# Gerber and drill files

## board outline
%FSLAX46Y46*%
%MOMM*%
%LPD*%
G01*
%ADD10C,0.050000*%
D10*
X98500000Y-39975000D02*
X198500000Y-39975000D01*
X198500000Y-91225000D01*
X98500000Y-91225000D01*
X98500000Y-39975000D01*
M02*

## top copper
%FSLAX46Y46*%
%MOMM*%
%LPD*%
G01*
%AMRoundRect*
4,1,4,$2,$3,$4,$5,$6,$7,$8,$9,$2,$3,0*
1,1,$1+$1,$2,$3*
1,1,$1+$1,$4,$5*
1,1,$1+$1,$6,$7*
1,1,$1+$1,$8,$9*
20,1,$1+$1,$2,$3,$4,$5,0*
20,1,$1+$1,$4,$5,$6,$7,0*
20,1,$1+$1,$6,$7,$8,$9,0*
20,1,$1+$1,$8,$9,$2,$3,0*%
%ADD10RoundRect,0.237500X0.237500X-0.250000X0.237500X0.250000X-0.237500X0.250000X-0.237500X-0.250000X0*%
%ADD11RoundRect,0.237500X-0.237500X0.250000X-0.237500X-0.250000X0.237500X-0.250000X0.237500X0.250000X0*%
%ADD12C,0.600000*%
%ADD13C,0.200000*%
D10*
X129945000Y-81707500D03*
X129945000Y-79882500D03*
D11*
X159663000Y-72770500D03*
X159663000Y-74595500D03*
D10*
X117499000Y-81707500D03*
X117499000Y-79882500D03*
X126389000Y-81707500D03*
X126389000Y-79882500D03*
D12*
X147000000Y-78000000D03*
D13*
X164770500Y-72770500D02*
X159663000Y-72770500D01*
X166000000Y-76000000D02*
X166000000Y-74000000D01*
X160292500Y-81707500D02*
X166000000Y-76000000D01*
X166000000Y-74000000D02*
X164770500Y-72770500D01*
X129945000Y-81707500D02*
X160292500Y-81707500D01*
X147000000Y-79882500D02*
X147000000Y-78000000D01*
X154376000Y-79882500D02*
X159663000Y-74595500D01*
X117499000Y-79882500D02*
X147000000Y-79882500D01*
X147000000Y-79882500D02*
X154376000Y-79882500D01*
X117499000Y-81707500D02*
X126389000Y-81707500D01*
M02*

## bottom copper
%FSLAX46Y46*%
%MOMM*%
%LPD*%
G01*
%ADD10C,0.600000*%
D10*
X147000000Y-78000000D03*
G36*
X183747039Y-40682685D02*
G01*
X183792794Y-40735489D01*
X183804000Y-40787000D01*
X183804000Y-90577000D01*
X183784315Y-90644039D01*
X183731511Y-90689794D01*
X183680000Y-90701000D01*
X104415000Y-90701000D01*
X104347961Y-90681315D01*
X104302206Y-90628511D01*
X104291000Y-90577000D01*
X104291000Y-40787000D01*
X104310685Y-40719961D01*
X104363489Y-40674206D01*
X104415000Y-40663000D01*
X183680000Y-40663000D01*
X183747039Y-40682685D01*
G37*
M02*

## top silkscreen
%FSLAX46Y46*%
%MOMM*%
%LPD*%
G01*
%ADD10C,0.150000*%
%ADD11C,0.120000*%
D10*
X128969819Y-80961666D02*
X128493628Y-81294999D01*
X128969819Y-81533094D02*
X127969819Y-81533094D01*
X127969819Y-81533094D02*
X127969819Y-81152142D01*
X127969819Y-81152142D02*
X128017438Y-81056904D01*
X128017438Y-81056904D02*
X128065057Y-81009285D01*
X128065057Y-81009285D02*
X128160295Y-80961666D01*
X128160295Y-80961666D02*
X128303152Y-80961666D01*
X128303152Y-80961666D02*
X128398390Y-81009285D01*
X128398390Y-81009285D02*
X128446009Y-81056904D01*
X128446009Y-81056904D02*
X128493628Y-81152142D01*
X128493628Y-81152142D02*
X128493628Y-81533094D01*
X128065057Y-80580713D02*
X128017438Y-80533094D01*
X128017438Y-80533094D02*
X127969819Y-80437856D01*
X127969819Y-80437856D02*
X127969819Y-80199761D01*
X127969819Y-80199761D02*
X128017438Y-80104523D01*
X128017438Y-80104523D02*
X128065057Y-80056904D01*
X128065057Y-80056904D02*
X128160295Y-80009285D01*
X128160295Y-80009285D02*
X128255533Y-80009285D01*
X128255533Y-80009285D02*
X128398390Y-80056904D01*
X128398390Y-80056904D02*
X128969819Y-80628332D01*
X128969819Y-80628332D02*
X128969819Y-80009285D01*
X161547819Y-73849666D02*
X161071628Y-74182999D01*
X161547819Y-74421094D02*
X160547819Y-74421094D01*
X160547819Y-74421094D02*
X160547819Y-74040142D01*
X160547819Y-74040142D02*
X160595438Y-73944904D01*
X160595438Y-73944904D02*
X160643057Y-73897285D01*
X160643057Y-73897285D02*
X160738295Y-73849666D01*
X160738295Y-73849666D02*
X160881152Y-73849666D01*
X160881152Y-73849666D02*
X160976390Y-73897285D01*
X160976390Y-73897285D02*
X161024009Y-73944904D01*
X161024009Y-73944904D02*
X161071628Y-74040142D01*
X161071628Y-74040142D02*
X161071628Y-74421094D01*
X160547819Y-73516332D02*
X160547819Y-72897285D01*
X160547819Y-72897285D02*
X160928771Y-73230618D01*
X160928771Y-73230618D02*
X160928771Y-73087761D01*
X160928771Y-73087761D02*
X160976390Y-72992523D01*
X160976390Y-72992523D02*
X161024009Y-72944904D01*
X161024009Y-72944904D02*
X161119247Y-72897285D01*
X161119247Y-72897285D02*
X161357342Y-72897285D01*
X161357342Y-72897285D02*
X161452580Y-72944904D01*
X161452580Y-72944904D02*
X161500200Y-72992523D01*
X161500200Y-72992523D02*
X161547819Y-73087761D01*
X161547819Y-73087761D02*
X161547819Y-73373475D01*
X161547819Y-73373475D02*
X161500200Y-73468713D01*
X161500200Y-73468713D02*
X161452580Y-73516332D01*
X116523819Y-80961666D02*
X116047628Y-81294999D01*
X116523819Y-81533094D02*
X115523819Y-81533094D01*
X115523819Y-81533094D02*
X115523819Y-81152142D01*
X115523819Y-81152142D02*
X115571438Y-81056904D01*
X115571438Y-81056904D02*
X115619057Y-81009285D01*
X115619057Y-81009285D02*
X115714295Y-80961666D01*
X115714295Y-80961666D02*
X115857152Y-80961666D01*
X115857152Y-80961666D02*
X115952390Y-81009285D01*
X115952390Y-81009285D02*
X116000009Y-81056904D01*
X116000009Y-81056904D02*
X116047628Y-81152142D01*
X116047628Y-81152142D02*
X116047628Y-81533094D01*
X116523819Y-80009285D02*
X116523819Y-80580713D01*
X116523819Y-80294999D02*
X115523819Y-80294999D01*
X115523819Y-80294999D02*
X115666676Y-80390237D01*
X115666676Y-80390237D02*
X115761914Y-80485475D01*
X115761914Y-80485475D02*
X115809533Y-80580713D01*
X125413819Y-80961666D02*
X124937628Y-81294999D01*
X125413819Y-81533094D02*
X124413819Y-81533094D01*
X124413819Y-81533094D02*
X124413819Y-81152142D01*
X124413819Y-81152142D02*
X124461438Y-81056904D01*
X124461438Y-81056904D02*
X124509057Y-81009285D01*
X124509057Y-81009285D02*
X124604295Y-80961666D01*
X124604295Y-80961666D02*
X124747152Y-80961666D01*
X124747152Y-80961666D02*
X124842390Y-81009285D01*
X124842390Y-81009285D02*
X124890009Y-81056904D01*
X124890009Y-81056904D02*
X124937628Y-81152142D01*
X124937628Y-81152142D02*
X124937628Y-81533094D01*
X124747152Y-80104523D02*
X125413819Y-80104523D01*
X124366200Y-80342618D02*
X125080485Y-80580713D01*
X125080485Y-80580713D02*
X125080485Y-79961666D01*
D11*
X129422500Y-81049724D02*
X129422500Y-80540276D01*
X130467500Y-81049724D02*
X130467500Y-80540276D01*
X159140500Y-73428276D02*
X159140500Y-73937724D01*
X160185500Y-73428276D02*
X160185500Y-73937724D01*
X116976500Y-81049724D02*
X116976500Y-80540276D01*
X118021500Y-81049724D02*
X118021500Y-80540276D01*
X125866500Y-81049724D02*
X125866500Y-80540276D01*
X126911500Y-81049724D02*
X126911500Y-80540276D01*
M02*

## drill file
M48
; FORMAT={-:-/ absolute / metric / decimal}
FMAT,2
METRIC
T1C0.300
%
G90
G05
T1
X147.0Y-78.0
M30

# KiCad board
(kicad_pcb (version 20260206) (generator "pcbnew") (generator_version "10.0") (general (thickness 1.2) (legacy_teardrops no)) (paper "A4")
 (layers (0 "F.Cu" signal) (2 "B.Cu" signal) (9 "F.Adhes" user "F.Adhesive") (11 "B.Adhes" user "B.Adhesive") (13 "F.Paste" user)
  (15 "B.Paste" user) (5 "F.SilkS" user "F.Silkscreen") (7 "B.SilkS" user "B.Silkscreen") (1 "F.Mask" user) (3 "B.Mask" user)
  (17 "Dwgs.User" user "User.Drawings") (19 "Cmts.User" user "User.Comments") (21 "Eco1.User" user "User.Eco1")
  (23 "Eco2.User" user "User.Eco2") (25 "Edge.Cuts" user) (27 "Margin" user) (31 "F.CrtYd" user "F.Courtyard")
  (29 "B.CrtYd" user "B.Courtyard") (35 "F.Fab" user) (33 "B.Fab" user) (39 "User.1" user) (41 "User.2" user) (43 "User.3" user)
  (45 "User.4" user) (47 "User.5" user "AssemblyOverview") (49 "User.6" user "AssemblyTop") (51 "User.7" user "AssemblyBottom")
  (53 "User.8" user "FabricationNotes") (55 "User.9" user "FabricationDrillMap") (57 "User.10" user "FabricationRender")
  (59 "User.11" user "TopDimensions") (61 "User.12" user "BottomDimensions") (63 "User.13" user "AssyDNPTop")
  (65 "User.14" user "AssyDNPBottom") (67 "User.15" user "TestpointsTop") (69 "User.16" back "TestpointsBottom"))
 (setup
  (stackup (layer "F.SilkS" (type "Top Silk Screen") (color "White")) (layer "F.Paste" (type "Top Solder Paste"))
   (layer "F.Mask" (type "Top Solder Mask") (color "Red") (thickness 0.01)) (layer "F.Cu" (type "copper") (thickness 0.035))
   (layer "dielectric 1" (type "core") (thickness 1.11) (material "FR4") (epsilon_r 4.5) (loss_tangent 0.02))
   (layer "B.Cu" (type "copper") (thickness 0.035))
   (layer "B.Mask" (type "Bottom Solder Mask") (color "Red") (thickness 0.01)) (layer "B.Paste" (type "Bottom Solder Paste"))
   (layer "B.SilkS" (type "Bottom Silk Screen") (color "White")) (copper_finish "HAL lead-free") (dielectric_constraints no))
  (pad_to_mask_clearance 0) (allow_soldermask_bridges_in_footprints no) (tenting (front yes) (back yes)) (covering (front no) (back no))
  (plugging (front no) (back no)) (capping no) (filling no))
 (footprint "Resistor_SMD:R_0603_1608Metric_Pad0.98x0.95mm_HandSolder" (layer "F.Cu") (at 129.945 80.795 90)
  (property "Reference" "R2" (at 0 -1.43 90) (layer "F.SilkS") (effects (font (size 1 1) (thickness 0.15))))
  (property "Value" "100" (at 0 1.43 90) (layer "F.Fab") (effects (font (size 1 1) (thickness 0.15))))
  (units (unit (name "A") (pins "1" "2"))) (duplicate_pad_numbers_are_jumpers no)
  (fp_line (start -0.254724 -0.5225) (end 0.254724 -0.5225) (stroke (width 0.12) (type solid)) (layer "F.SilkS"))
  (fp_line (start -0.254724 0.5225) (end 0.254724 0.5225) (stroke (width 0.12) (type solid)) (layer "F.SilkS"))
  (pad "1" smd roundrect (at -0.9125 0 90) (size 0.975 0.95) (layers "F.Cu" "F.Mask" "F.Paste") (roundrect_rratio 0.25)
   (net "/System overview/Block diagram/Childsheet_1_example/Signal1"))
  (pad "2" smd roundrect (at 0.9125 0 90) (size 0.975 0.95) (layers "F.Cu" "F.Mask" "F.Paste") (roundrect_rratio 0.25) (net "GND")))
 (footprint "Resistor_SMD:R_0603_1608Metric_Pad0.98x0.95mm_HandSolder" (layer "F.Cu") (at 159.663 73.683 -90)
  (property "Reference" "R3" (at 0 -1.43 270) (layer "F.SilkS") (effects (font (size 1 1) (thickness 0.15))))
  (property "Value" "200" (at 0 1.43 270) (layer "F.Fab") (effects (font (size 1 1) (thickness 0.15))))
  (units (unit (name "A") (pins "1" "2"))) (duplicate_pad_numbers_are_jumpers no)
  (fp_line (start -0.254724 0.5225) (end 0.254724 0.5225) (stroke (width 0.12) (type solid)) (layer "F.SilkS"))
  (fp_line (start -0.254724 -0.5225) (end 0.254724 -0.5225) (stroke (width 0.12) (type solid)) (layer "F.SilkS"))
  (pad "1" smd roundrect (at -0.9125 0 270) (size 0.975 0.95) (layers "F.Cu" "F.Mask" "F.Paste") (roundrect_rratio 0.25)
   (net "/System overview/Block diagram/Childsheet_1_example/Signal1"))
  (pad "2" smd roundrect (at 0.9125 0 270) (size 0.975 0.95) (layers "F.Cu" "F.Mask" "F.Paste") (roundrect_rratio 0.25) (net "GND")))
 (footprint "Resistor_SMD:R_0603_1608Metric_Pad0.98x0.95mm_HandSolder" (layer "F.Cu") (at 117.499 80.795 90)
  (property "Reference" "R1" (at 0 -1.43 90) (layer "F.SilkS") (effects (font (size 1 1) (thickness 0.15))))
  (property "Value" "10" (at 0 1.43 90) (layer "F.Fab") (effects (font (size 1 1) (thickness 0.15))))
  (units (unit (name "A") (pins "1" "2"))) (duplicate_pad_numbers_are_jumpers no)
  (fp_line (start -0.254724 -0.5225) (end 0.254724 -0.5225) (stroke (width 0.12) (type solid)) (layer "F.SilkS"))
  (fp_line (start -0.254724 0.5225) (end 0.254724 0.5225) (stroke (width 0.12) (type solid)) (layer "F.SilkS"))
  (pad "1" smd roundrect (at -0.9125 0 90) (size 0.975 0.95) (layers "F.Cu" "F.Mask" "F.Paste") (roundrect_rratio 0.25)
   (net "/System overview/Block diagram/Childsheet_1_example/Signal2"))
  (pad "2" smd roundrect (at 0.9125 0 90) (size 0.975 0.95) (layers "F.Cu" "F.Mask" "F.Paste") (roundrect_rratio 0.25) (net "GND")))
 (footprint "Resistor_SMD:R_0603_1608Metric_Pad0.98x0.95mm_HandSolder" (layer "F.Cu") (at 126.389 80.795 90)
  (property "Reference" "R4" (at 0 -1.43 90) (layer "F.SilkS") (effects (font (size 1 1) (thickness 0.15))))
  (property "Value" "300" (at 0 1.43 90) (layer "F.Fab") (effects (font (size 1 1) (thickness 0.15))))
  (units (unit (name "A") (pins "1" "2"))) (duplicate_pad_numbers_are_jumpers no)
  (fp_line (start -0.254724 -0.5225) (end 0.254724 -0.5225) (stroke (width 0.12) (type solid)) (layer "F.SilkS"))
  (fp_line (start -0.254724 0.5225) (end 0.254724 0.5225) (stroke (width 0.12) (type solid)) (layer "F.SilkS"))
  (pad "1" smd roundrect (at -0.9125 0 90) (size 0.975 0.95) (layers "F.Cu" "F.Mask" "F.Paste") (roundrect_rratio 0.25)
   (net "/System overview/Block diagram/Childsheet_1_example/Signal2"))
  (pad "2" smd roundrect (at 0.9125 0 90) (size 0.975 0.95) (layers "F.Cu" "F.Mask" "F.Paste") (roundrect_rratio 0.25) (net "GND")))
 (gr_rect (start 98.5 39.975) (end 198.5 91.225) (stroke (width 0.05) (type solid)) (fill no) (layer "Edge.Cuts"))
 (segment (start 164.7705 72.7705) (end 159.663 72.7705) (width 0.2) (layer "F.Cu")
  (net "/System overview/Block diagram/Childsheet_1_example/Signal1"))
 (segment (start 166 76) (end 166 74) (width 0.2) (layer "F.Cu") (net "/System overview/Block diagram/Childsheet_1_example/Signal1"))
 (segment (start 160.2925 81.7075) (end 166 76) (width 0.2) (layer "F.Cu")
  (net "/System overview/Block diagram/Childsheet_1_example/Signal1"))
 (segment (start 166 74) (end 164.7705 72.7705) (width 0.2) (layer "F.Cu")
  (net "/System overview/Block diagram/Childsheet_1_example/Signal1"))
 (segment (start 129.945 81.7075) (end 160.2925 81.7075) (width 0.2) (layer "F.Cu")
  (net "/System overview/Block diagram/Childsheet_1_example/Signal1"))
 (segment (start 147 79.8825) (end 147 78) (width 0.2) (layer "F.Cu") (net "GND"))
 (segment (start 154.376 79.8825) (end 159.663 74.5955) (width 0.2) (layer "F.Cu") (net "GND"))
 (segment (start 117.499 79.8825) (end 147 79.8825) (width 0.2) (layer "F.Cu") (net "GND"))
 (segment (start 147 79.8825) (end 154.376 79.8825) (width 0.2) (layer "F.Cu") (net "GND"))
 (via (at 147 78) (size 0.6) (drill 0.3) (layers "F.Cu" "B.Cu") (free yes) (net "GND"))
 (segment (start 117.499 81.7075) (end 126.389 81.7075) (width 0.2) (layer "F.Cu")
  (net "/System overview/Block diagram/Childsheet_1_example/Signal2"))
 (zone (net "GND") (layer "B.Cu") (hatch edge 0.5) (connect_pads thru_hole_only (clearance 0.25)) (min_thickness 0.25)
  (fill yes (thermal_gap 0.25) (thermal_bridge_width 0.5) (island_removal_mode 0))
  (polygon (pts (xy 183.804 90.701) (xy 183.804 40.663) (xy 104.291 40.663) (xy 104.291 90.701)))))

